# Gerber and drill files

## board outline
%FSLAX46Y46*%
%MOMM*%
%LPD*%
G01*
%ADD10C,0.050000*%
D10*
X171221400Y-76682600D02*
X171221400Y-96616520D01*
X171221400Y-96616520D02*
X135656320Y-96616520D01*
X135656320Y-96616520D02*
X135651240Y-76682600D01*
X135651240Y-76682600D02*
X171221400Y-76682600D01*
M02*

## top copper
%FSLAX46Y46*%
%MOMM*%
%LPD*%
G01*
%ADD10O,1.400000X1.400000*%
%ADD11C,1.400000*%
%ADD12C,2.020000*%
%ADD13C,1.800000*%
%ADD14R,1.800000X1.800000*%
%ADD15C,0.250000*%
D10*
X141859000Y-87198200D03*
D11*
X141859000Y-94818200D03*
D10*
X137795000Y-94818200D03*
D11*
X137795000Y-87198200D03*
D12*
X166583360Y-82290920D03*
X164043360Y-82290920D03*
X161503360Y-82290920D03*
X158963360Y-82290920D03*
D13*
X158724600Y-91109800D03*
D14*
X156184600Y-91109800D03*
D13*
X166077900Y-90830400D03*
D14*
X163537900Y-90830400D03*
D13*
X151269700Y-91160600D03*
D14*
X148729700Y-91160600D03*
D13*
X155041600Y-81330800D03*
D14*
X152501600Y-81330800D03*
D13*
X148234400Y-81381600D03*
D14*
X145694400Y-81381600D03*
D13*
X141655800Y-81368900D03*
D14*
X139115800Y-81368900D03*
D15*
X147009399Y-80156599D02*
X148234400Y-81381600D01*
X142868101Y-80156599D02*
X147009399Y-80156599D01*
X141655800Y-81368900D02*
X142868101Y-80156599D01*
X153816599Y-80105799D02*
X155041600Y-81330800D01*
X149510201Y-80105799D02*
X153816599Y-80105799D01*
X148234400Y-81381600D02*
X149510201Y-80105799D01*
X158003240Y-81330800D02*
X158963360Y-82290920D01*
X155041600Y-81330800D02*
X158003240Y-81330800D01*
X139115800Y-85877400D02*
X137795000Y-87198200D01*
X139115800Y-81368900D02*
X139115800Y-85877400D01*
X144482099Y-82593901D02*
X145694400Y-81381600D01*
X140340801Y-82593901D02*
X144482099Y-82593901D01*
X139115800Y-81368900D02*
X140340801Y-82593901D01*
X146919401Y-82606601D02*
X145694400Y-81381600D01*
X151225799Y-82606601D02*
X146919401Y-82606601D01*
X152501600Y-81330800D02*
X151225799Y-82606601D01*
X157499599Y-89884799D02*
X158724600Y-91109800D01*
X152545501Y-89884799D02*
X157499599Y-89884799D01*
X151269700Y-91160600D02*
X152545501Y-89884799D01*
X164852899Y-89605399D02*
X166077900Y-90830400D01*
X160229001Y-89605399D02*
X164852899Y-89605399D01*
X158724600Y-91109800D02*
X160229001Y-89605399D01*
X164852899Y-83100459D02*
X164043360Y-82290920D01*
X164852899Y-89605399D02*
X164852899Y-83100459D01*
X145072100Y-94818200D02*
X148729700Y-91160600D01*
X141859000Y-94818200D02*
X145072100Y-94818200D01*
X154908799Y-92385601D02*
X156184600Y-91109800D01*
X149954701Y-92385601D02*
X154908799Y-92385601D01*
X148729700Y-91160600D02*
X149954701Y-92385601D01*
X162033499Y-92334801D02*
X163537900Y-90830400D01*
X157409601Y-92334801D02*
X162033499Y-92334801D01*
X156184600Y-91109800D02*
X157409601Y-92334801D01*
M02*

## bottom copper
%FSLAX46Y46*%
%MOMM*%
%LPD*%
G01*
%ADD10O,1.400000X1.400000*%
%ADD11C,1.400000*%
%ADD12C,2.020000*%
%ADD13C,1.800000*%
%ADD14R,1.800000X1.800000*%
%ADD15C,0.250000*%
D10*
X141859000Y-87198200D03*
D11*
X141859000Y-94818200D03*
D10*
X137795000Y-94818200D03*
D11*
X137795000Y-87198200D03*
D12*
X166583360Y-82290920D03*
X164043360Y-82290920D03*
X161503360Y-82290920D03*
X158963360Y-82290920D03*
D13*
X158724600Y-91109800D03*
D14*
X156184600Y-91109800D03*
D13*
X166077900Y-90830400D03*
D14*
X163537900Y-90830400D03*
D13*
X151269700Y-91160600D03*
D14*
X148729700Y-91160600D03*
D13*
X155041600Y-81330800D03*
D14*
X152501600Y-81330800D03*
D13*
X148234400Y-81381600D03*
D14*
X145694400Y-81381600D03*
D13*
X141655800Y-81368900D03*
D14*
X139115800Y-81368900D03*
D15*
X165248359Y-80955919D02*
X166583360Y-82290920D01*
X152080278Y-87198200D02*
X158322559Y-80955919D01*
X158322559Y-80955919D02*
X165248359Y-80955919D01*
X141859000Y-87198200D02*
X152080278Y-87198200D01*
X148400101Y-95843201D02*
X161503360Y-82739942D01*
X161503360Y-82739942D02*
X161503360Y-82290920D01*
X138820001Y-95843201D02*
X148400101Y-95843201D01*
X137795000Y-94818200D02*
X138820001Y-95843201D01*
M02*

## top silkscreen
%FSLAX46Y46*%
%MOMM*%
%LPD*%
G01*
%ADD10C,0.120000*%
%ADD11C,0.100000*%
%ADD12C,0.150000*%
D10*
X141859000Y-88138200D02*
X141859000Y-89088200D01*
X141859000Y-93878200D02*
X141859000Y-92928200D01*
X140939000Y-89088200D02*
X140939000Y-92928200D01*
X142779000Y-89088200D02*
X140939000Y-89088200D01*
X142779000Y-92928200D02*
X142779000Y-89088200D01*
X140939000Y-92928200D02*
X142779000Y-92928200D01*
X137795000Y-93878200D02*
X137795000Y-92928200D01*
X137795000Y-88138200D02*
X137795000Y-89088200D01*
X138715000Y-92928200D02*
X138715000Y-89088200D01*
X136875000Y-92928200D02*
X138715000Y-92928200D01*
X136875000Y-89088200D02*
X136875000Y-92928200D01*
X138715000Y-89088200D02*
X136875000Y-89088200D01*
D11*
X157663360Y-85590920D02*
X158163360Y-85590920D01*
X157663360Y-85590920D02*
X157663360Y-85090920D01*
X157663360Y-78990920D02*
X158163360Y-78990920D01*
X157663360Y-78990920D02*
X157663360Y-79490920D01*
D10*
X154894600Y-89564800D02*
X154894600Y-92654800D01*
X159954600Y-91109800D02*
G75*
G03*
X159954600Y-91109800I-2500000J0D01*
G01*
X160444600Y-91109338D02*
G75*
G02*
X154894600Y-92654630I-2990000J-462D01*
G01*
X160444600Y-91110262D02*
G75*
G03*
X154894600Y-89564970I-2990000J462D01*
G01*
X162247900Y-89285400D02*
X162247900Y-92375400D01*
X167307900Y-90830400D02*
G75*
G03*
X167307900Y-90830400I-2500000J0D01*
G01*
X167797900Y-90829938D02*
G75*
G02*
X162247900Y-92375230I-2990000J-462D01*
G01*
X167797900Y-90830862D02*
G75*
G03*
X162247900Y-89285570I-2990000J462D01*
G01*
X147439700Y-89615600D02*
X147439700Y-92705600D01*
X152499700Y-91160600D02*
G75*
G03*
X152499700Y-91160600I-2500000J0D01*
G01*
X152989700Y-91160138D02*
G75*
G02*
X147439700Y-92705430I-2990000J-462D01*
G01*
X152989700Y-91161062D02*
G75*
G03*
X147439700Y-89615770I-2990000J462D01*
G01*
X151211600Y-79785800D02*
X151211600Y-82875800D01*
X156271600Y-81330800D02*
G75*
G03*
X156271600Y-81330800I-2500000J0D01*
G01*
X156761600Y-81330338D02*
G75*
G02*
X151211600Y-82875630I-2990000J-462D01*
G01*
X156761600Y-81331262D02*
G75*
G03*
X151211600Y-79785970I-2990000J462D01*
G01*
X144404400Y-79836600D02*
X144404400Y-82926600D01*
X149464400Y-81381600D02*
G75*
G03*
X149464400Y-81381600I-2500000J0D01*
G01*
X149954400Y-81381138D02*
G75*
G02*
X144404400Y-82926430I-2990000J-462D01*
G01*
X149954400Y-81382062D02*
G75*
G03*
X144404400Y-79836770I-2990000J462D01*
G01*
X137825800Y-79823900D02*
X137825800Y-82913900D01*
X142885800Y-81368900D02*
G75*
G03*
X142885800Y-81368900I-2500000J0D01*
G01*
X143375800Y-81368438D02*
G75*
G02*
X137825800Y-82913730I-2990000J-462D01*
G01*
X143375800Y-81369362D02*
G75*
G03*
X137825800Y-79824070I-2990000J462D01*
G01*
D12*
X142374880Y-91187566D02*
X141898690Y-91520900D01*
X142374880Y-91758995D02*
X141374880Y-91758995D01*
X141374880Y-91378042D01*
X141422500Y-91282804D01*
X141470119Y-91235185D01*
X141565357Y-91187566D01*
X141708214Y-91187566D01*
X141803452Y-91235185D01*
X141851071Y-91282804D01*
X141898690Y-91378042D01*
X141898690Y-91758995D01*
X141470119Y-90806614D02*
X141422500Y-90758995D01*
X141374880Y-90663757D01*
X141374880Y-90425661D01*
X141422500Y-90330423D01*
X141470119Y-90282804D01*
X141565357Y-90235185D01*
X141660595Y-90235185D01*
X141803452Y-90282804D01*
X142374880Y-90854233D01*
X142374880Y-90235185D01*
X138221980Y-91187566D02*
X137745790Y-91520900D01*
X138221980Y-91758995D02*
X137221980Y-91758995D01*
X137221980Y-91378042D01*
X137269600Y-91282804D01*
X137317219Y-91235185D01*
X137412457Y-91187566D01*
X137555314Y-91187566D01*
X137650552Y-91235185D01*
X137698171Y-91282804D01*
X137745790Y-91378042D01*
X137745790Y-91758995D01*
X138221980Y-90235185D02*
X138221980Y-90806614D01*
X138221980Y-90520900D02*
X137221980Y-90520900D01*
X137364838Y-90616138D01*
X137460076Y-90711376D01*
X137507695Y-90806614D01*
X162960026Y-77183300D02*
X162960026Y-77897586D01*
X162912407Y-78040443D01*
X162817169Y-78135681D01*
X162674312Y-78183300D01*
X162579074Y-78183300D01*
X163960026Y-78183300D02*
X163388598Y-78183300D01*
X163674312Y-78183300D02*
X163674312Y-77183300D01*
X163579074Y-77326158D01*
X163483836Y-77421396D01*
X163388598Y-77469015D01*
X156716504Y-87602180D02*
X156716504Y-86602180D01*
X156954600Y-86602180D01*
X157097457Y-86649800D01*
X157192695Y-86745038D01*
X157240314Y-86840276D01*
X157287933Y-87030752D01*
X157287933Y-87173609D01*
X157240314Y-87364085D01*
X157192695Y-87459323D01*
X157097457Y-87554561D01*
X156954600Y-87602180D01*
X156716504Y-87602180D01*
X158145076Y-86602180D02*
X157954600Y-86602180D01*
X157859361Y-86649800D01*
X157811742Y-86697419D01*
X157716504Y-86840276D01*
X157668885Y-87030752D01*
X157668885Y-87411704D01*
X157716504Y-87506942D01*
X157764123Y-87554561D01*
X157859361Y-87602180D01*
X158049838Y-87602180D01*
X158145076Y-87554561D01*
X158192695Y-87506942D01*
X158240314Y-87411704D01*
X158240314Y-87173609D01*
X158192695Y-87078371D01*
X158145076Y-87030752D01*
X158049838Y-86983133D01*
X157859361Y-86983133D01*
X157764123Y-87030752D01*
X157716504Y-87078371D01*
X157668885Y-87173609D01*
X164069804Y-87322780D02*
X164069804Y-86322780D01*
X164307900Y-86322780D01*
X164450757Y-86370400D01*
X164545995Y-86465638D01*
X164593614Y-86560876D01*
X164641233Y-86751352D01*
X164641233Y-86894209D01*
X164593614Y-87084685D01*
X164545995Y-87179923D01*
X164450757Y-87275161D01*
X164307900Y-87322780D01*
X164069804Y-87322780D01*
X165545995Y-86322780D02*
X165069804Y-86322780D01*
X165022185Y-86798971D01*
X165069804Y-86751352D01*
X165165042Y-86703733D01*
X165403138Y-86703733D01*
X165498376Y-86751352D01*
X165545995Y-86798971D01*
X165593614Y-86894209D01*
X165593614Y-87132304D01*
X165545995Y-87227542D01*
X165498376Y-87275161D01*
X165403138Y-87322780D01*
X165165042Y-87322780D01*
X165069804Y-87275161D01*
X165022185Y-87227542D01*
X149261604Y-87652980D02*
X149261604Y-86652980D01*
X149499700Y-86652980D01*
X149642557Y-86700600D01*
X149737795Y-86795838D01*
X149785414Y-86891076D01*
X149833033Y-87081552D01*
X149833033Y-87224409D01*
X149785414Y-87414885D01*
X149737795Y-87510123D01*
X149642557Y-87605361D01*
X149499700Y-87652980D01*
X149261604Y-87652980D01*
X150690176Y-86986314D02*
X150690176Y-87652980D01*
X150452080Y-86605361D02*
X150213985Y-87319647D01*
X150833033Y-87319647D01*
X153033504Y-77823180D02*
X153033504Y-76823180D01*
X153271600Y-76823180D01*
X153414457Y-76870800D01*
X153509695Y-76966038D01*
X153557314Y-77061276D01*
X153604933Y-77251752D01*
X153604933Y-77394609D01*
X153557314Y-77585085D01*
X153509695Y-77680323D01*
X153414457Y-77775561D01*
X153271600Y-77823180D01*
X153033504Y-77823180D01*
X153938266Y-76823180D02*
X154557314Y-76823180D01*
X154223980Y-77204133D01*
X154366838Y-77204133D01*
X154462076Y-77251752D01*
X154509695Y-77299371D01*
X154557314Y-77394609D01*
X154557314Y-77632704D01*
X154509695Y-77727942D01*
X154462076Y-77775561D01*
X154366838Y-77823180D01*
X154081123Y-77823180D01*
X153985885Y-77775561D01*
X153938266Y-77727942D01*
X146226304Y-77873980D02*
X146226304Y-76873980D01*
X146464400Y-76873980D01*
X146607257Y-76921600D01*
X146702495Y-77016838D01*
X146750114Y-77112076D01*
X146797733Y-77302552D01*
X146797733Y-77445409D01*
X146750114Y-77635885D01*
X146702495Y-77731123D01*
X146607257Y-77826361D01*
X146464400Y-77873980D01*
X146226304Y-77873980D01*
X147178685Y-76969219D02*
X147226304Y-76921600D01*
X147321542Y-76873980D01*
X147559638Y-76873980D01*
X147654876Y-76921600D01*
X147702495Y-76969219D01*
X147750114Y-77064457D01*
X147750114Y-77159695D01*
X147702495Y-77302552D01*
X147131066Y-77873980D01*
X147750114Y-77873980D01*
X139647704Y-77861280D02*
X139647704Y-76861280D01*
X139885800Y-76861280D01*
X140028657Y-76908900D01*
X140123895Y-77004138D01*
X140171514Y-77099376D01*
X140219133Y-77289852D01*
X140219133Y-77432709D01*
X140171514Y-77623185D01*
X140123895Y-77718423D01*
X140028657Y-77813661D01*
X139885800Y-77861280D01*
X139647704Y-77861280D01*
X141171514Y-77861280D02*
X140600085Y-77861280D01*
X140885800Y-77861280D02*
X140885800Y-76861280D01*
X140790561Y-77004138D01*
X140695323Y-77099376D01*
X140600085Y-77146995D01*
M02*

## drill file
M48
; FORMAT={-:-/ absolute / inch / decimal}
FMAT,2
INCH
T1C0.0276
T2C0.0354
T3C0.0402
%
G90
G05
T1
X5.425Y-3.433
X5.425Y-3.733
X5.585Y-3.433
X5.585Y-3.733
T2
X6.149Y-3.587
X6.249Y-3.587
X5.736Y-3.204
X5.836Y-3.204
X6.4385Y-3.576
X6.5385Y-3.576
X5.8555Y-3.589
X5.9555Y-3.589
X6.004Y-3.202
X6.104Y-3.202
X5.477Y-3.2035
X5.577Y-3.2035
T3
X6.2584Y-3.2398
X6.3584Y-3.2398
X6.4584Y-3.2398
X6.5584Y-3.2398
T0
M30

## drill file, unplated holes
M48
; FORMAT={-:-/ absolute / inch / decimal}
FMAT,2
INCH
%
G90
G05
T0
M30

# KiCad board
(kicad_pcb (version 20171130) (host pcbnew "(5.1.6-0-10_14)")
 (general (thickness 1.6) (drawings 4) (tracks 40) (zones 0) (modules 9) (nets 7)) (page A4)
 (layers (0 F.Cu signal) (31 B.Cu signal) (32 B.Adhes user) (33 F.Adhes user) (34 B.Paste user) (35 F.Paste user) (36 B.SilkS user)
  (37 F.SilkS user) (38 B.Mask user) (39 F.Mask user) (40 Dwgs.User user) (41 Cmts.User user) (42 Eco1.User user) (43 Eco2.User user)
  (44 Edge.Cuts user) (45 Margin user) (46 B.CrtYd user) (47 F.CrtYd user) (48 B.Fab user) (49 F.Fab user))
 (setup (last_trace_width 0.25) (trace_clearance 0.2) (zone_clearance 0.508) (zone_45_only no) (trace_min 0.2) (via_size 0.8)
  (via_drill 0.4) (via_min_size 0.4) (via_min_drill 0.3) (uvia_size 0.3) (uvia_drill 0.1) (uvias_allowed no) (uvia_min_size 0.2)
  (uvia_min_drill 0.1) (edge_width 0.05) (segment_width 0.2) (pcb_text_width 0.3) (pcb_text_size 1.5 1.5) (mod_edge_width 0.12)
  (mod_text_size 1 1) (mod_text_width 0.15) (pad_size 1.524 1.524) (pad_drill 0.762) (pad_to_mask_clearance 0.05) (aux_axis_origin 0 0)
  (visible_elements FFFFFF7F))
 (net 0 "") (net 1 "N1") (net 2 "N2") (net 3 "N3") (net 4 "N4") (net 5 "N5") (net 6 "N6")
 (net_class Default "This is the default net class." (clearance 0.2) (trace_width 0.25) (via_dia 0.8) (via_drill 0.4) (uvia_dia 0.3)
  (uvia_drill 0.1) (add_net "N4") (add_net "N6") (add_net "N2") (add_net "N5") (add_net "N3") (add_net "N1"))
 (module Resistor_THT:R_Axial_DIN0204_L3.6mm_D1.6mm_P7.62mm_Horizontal (layer F.Cu) (at 141.859 94.8182 90)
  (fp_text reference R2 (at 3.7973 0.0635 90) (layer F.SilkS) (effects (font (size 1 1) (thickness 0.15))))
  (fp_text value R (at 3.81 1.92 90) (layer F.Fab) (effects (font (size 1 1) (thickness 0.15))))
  (fp_line (start 6.68 0) (end 5.73 0) (layer F.SilkS) (width 0.12))
  (fp_line (start 0.94 0) (end 1.89 0) (layer F.SilkS) (width 0.12))
  (fp_line (start 5.73 -0.92) (end 1.89 -0.92) (layer F.SilkS) (width 0.12))
  (fp_line (start 5.73 0.92) (end 5.73 -0.92) (layer F.SilkS) (width 0.12))
  (fp_line (start 1.89 0.92) (end 5.73 0.92) (layer F.SilkS) (width 0.12))
  (fp_line (start 1.89 -0.92) (end 1.89 0.92) (layer F.SilkS) (width 0.12))
  (pad 2 thru_hole oval (at 7.62 0 90) (size 1.4 1.4) (drill 0.7) (layers *.Cu *.Mask) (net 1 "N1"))
  (pad 1 thru_hole circle (at 0 0 90) (size 1.4 1.4) (drill 0.7) (layers *.Cu *.Mask) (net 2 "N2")))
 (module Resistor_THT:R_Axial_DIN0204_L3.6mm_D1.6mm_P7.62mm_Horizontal (layer F.Cu) (at 137.795 87.1982 270)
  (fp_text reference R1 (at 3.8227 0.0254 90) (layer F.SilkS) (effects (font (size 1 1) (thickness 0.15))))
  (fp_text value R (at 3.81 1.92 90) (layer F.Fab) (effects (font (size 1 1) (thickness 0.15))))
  (fp_line (start 6.68 0) (end 5.73 0) (layer F.SilkS) (width 0.12))
  (fp_line (start 0.94 0) (end 1.89 0) (layer F.SilkS) (width 0.12))
  (fp_line (start 5.73 -0.92) (end 1.89 -0.92) (layer F.SilkS) (width 0.12))
  (fp_line (start 5.73 0.92) (end 5.73 -0.92) (layer F.SilkS) (width 0.12))
  (fp_line (start 1.89 0.92) (end 5.73 0.92) (layer F.SilkS) (width 0.12))
  (fp_line (start 1.89 -0.92) (end 1.89 0.92) (layer F.SilkS) (width 0.12))
  (pad 2 thru_hole oval (at 7.62 0 270) (size 1.4 1.4) (drill 0.7) (layers *.Cu *.Mask) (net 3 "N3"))
  (pad 1 thru_hole circle (at 0 0 270) (size 1.4 1.4) (drill 0.7) (layers *.Cu *.Mask) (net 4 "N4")))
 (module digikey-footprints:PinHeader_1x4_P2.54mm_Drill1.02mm (layer F.Cu) (at 158.96336 82.29092)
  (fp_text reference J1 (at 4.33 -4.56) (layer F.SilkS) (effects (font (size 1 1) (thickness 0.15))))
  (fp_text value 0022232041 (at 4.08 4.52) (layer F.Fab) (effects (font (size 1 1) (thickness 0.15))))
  (fp_line (start -1.3 3.3) (end -0.8 3.3) (layer F.SilkS) (width 0.1))
  (fp_line (start -1.3 3.3) (end -1.3 2.8) (layer F.SilkS) (width 0.1))
  (fp_line (start -1.3 -3.3) (end -0.8 -3.3) (layer F.SilkS) (width 0.1))
  (fp_line (start -1.3 -3.3) (end -1.3 -2.8) (layer F.SilkS) (width 0.1))
  (pad 4 thru_hole circle (at 7.62 0) (size 2.02 2.02) (drill 1.02) (layers *.Cu *.Mask) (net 1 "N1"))
  (pad 3 thru_hole circle (at 5.08 0) (size 2.02 2.02) (drill 1.02) (layers *.Cu *.Mask) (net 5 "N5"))
  (pad 2 thru_hole circle (at 2.54 0) (size 2.02 2.02) (drill 1.02) (layers *.Cu *.Mask) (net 3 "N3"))
  (pad 1 thru_hole circle (at 0 0) (size 2.02 2.02) (drill 1.02) (layers *.Cu *.Mask) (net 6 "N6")))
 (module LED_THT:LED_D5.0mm (layer F.Cu) (at 156.1846 91.1098)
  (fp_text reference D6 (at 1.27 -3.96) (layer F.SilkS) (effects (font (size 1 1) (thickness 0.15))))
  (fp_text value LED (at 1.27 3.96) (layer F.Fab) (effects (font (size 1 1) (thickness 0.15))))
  (fp_line (start -1.29 -1.545) (end -1.29 1.545) (layer F.SilkS) (width 0.12))
  (fp_circle (center 1.27 0) (end 3.77 0) (layer F.SilkS) (width 0.12))
  (fp_arc (start 1.27 0) (end -1.29 1.54483) (angle -148.9) (layer F.SilkS) (width 0.12))
  (fp_arc (start 1.27 0) (end -1.29 -1.54483) (angle 148.9) (layer F.SilkS) (width 0.12))
  (pad 2 thru_hole circle (at 2.54 0) (size 1.8 1.8) (drill 0.9) (layers *.Cu *.Mask) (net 5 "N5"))
  (pad 1 thru_hole rect (at 0 0) (size 1.8 1.8) (drill 0.9) (layers *.Cu *.Mask) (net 2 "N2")))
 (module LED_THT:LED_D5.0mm (layer F.Cu) (at 163.5379 90.8304)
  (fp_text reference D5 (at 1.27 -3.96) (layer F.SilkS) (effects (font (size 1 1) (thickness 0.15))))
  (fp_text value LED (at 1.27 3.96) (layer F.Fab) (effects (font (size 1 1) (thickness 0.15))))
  (fp_line (start -1.29 -1.545) (end -1.29 1.545) (layer F.SilkS) (width 0.12))
  (fp_circle (center 1.27 0) (end 3.77 0) (layer F.SilkS) (width 0.12))
  (fp_arc (start 1.27 0) (end -1.29 1.54483) (angle -148.9) (layer F.SilkS) (width 0.12))
  (fp_arc (start 1.27 0) (end -1.29 -1.54483) (angle 148.9) (layer F.SilkS) (width 0.12))
  (pad 2 thru_hole circle (at 2.54 0) (size 1.8 1.8) (drill 0.9) (layers *.Cu *.Mask) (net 5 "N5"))
  (pad 1 thru_hole rect (at 0 0) (size 1.8 1.8) (drill 0.9) (layers *.Cu *.Mask) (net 2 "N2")))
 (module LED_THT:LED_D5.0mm (layer F.Cu) (at 148.7297 91.1606)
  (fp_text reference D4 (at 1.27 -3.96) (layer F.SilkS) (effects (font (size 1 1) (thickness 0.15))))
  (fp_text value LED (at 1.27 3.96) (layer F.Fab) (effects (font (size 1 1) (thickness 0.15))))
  (fp_line (start -1.29 -1.545) (end -1.29 1.545) (layer F.SilkS) (width 0.12))
  (fp_circle (center 1.27 0) (end 3.77 0) (layer F.SilkS) (width 0.12))
  (fp_arc (start 1.27 0) (end -1.29 1.54483) (angle -148.9) (layer F.SilkS) (width 0.12))
  (fp_arc (start 1.27 0) (end -1.29 -1.54483) (angle 148.9) (layer F.SilkS) (width 0.12))
  (pad 2 thru_hole circle (at 2.54 0) (size 1.8 1.8) (drill 0.9) (layers *.Cu *.Mask) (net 5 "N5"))
  (pad 1 thru_hole rect (at 0 0) (size 1.8 1.8) (drill 0.9) (layers *.Cu *.Mask) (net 2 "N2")))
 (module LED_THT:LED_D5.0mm (layer F.Cu) (at 152.5016 81.3308)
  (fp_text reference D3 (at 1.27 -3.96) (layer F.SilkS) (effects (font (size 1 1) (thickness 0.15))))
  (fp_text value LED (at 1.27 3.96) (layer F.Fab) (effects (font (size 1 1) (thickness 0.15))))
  (fp_line (start -1.29 -1.545) (end -1.29 1.545) (layer F.SilkS) (width 0.12))
  (fp_circle (center 1.27 0) (end 3.77 0) (layer F.SilkS) (width 0.12))
  (fp_arc (start 1.27 0) (end -1.29 1.54483) (angle -148.9) (layer F.SilkS) (width 0.12))
  (fp_arc (start 1.27 0) (end -1.29 -1.54483) (angle 148.9) (layer F.SilkS) (width 0.12))
  (pad 2 thru_hole circle (at 2.54 0) (size 1.8 1.8) (drill 0.9) (layers *.Cu *.Mask) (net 6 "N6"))
  (pad 1 thru_hole rect (at 0 0) (size 1.8 1.8) (drill 0.9) (layers *.Cu *.Mask) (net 4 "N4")))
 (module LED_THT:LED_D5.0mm (layer F.Cu) (at 145.6944 81.3816)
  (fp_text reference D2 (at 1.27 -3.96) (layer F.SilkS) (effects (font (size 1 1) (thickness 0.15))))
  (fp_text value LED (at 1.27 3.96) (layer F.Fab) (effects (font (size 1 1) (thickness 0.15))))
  (fp_line (start -1.29 -1.545) (end -1.29 1.545) (layer F.SilkS) (width 0.12))
  (fp_circle (center 1.27 0) (end 3.77 0) (layer F.SilkS) (width 0.12))
  (fp_arc (start 1.27 0) (end -1.29 1.54483) (angle -148.9) (layer F.SilkS) (width 0.12))
  (fp_arc (start 1.27 0) (end -1.29 -1.54483) (angle 148.9) (layer F.SilkS) (width 0.12))
  (pad 2 thru_hole circle (at 2.54 0) (size 1.8 1.8) (drill 0.9) (layers *.Cu *.Mask) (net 6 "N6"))
  (pad 1 thru_hole rect (at 0 0) (size 1.8 1.8) (drill 0.9) (layers *.Cu *.Mask) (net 4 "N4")))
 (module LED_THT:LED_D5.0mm (layer F.Cu) (at 139.1158 81.3689)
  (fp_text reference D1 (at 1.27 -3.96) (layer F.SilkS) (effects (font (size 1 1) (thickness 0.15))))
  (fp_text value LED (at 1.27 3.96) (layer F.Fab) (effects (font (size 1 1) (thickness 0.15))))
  (fp_line (start -1.29 -1.545) (end -1.29 1.545) (layer F.SilkS) (width 0.12))
  (fp_circle (center 1.27 0) (end 3.77 0) (layer F.SilkS) (width 0.12))
  (fp_arc (start 1.27 0) (end -1.29 1.54483) (angle -148.9) (layer F.SilkS) (width 0.12))
  (fp_arc (start 1.27 0) (end -1.29 -1.54483) (angle 148.9) (layer F.SilkS) (width 0.12))
  (pad 2 thru_hole circle (at 2.54 0) (size 1.8 1.8) (drill 0.9) (layers *.Cu *.Mask) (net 6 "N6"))
  (pad 1 thru_hole rect (at 0 0) (size 1.8 1.8) (drill 0.9) (layers *.Cu *.Mask) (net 4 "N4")))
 (gr_line (start 171.2214 76.6826) (end 171.2214 96.61652) (layer Edge.Cuts) (width 0.05))
 (gr_line (start 171.2214 96.61652) (end 135.65632 96.61652) (layer Edge.Cuts) (width 0.05))
 (gr_line (start 135.65632 96.61652) (end 135.65124 76.6826) (layer Edge.Cuts) (width 0.05))
 (gr_line (start 135.65124 76.6826) (end 171.2214 76.6826) (layer Edge.Cuts) (width 0.05))
 (segment (start 147.009399 80.156599) (end 148.2344 81.3816) (width 0.25) (layer F.Cu) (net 6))
 (segment (start 142.868101 80.156599) (end 147.009399 80.156599) (width 0.25) (layer F.Cu) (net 6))
 (segment (start 141.6558 81.3689) (end 142.868101 80.156599) (width 0.25) (layer F.Cu) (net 6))
 (segment (start 153.816599 80.105799) (end 155.0416 81.3308) (width 0.25) (layer F.Cu) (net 6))
 (segment (start 149.510201 80.105799) (end 153.816599 80.105799) (width 0.25) (layer F.Cu) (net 6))
 (segment (start 148.2344 81.3816) (end 149.510201 80.105799) (width 0.25) (layer F.Cu) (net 6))
 (segment (start 158.00324 81.3308) (end 158.96336 82.29092) (width 0.25) (layer F.Cu) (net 6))
 (segment (start 155.0416 81.3308) (end 158.00324 81.3308) (width 0.25) (layer F.Cu) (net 6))
 (segment (start 139.1158 85.8774) (end 137.795 87.1982) (width 0.25) (layer F.Cu) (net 4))
 (segment (start 139.1158 81.3689) (end 139.1158 85.8774) (width 0.25) (layer F.Cu) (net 4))
 (segment (start 144.482099 82.593901) (end 145.6944 81.3816) (width 0.25) (layer F.Cu) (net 4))
 (segment (start 140.340801 82.593901) (end 144.482099 82.593901) (width 0.25) (layer F.Cu) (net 4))
 (segment (start 139.1158 81.3689) (end 140.340801 82.593901) (width 0.25) (layer F.Cu) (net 4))
 (segment (start 146.919401 82.606601) (end 145.6944 81.3816) (width 0.25) (layer F.Cu) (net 4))
 (segment (start 151.225799 82.606601) (end 146.919401 82.606601) (width 0.25) (layer F.Cu) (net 4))
 (segment (start 152.5016 81.3308) (end 151.225799 82.606601) (width 0.25) (layer F.Cu) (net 4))
 (segment (start 157.499599 89.884799) (end 158.7246 91.1098) (width 0.25) (layer F.Cu) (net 5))
 (segment (start 152.545501 89.884799) (end 157.499599 89.884799) (width 0.25) (layer F.Cu) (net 5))
 (segment (start 151.2697 91.1606) (end 152.545501 89.884799) (width 0.25) (layer F.Cu) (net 5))
 (segment (start 164.852899 89.605399) (end 166.0779 90.8304) (width 0.25) (layer F.Cu) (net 5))
 (segment (start 160.229001 89.605399) (end 164.852899 89.605399) (width 0.25) (layer F.Cu) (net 5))
 (segment (start 158.7246 91.1098) (end 160.229001 89.605399) (width 0.25) (layer F.Cu) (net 5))
 (segment (start 164.852899 83.100459) (end 164.04336 82.29092) (width 0.25) (layer F.Cu) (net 5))
 (segment (start 164.852899 89.605399) (end 164.852899 83.100459) (width 0.25) (layer F.Cu) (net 5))
 (segment (start 145.0721 94.8182) (end 148.7297 91.1606) (width 0.25) (layer F.Cu) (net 2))
 (segment (start 141.859 94.8182) (end 145.0721 94.8182) (width 0.25) (layer F.Cu) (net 2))
 (segment (start 154.908799 92.385601) (end 156.1846 91.1098) (width 0.25) (layer F.Cu) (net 2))
 (segment (start 149.954701 92.385601) (end 154.908799 92.385601) (width 0.25) (layer F.Cu) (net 2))
 (segment (start 148.7297 91.1606) (end 149.954701 92.385601) (width 0.25) (layer F.Cu) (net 2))
 (segment (start 162.033499 92.334801) (end 163.5379 90.8304) (width 0.25) (layer F.Cu) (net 2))
 (segment (start 157.409601 92.334801) (end 162.033499 92.334801) (width 0.25) (layer F.Cu) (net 2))
 (segment (start 156.1846 91.1098) (end 157.409601 92.334801) (width 0.25) (layer F.Cu) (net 2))
 (segment (start 165.248359 80.955919) (end 166.58336 82.29092) (width 0.25) (layer B.Cu) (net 1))
 (segment (start 152.080278 87.1982) (end 158.322559 80.955919) (width 0.25) (layer B.Cu) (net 1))
 (segment (start 158.322559 80.955919) (end 165.248359 80.955919) (width 0.25) (layer B.Cu) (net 1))
 (segment (start 141.859 87.1982) (end 152.080278 87.1982) (width 0.25) (layer B.Cu) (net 1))
 (segment (start 148.400101 95.843201) (end 161.50336 82.739942) (width 0.25) (layer B.Cu) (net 3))
 (segment (start 161.50336 82.739942) (end 161.50336 82.29092) (width 0.25) (layer B.Cu) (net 3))
 (segment (start 138.820001 95.843201) (end 148.400101 95.843201) (width 0.25) (layer B.Cu) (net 3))
 (segment (start 137.795 94.8182) (end 138.820001 95.843201) (width 0.25) (layer B.Cu) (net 3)))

